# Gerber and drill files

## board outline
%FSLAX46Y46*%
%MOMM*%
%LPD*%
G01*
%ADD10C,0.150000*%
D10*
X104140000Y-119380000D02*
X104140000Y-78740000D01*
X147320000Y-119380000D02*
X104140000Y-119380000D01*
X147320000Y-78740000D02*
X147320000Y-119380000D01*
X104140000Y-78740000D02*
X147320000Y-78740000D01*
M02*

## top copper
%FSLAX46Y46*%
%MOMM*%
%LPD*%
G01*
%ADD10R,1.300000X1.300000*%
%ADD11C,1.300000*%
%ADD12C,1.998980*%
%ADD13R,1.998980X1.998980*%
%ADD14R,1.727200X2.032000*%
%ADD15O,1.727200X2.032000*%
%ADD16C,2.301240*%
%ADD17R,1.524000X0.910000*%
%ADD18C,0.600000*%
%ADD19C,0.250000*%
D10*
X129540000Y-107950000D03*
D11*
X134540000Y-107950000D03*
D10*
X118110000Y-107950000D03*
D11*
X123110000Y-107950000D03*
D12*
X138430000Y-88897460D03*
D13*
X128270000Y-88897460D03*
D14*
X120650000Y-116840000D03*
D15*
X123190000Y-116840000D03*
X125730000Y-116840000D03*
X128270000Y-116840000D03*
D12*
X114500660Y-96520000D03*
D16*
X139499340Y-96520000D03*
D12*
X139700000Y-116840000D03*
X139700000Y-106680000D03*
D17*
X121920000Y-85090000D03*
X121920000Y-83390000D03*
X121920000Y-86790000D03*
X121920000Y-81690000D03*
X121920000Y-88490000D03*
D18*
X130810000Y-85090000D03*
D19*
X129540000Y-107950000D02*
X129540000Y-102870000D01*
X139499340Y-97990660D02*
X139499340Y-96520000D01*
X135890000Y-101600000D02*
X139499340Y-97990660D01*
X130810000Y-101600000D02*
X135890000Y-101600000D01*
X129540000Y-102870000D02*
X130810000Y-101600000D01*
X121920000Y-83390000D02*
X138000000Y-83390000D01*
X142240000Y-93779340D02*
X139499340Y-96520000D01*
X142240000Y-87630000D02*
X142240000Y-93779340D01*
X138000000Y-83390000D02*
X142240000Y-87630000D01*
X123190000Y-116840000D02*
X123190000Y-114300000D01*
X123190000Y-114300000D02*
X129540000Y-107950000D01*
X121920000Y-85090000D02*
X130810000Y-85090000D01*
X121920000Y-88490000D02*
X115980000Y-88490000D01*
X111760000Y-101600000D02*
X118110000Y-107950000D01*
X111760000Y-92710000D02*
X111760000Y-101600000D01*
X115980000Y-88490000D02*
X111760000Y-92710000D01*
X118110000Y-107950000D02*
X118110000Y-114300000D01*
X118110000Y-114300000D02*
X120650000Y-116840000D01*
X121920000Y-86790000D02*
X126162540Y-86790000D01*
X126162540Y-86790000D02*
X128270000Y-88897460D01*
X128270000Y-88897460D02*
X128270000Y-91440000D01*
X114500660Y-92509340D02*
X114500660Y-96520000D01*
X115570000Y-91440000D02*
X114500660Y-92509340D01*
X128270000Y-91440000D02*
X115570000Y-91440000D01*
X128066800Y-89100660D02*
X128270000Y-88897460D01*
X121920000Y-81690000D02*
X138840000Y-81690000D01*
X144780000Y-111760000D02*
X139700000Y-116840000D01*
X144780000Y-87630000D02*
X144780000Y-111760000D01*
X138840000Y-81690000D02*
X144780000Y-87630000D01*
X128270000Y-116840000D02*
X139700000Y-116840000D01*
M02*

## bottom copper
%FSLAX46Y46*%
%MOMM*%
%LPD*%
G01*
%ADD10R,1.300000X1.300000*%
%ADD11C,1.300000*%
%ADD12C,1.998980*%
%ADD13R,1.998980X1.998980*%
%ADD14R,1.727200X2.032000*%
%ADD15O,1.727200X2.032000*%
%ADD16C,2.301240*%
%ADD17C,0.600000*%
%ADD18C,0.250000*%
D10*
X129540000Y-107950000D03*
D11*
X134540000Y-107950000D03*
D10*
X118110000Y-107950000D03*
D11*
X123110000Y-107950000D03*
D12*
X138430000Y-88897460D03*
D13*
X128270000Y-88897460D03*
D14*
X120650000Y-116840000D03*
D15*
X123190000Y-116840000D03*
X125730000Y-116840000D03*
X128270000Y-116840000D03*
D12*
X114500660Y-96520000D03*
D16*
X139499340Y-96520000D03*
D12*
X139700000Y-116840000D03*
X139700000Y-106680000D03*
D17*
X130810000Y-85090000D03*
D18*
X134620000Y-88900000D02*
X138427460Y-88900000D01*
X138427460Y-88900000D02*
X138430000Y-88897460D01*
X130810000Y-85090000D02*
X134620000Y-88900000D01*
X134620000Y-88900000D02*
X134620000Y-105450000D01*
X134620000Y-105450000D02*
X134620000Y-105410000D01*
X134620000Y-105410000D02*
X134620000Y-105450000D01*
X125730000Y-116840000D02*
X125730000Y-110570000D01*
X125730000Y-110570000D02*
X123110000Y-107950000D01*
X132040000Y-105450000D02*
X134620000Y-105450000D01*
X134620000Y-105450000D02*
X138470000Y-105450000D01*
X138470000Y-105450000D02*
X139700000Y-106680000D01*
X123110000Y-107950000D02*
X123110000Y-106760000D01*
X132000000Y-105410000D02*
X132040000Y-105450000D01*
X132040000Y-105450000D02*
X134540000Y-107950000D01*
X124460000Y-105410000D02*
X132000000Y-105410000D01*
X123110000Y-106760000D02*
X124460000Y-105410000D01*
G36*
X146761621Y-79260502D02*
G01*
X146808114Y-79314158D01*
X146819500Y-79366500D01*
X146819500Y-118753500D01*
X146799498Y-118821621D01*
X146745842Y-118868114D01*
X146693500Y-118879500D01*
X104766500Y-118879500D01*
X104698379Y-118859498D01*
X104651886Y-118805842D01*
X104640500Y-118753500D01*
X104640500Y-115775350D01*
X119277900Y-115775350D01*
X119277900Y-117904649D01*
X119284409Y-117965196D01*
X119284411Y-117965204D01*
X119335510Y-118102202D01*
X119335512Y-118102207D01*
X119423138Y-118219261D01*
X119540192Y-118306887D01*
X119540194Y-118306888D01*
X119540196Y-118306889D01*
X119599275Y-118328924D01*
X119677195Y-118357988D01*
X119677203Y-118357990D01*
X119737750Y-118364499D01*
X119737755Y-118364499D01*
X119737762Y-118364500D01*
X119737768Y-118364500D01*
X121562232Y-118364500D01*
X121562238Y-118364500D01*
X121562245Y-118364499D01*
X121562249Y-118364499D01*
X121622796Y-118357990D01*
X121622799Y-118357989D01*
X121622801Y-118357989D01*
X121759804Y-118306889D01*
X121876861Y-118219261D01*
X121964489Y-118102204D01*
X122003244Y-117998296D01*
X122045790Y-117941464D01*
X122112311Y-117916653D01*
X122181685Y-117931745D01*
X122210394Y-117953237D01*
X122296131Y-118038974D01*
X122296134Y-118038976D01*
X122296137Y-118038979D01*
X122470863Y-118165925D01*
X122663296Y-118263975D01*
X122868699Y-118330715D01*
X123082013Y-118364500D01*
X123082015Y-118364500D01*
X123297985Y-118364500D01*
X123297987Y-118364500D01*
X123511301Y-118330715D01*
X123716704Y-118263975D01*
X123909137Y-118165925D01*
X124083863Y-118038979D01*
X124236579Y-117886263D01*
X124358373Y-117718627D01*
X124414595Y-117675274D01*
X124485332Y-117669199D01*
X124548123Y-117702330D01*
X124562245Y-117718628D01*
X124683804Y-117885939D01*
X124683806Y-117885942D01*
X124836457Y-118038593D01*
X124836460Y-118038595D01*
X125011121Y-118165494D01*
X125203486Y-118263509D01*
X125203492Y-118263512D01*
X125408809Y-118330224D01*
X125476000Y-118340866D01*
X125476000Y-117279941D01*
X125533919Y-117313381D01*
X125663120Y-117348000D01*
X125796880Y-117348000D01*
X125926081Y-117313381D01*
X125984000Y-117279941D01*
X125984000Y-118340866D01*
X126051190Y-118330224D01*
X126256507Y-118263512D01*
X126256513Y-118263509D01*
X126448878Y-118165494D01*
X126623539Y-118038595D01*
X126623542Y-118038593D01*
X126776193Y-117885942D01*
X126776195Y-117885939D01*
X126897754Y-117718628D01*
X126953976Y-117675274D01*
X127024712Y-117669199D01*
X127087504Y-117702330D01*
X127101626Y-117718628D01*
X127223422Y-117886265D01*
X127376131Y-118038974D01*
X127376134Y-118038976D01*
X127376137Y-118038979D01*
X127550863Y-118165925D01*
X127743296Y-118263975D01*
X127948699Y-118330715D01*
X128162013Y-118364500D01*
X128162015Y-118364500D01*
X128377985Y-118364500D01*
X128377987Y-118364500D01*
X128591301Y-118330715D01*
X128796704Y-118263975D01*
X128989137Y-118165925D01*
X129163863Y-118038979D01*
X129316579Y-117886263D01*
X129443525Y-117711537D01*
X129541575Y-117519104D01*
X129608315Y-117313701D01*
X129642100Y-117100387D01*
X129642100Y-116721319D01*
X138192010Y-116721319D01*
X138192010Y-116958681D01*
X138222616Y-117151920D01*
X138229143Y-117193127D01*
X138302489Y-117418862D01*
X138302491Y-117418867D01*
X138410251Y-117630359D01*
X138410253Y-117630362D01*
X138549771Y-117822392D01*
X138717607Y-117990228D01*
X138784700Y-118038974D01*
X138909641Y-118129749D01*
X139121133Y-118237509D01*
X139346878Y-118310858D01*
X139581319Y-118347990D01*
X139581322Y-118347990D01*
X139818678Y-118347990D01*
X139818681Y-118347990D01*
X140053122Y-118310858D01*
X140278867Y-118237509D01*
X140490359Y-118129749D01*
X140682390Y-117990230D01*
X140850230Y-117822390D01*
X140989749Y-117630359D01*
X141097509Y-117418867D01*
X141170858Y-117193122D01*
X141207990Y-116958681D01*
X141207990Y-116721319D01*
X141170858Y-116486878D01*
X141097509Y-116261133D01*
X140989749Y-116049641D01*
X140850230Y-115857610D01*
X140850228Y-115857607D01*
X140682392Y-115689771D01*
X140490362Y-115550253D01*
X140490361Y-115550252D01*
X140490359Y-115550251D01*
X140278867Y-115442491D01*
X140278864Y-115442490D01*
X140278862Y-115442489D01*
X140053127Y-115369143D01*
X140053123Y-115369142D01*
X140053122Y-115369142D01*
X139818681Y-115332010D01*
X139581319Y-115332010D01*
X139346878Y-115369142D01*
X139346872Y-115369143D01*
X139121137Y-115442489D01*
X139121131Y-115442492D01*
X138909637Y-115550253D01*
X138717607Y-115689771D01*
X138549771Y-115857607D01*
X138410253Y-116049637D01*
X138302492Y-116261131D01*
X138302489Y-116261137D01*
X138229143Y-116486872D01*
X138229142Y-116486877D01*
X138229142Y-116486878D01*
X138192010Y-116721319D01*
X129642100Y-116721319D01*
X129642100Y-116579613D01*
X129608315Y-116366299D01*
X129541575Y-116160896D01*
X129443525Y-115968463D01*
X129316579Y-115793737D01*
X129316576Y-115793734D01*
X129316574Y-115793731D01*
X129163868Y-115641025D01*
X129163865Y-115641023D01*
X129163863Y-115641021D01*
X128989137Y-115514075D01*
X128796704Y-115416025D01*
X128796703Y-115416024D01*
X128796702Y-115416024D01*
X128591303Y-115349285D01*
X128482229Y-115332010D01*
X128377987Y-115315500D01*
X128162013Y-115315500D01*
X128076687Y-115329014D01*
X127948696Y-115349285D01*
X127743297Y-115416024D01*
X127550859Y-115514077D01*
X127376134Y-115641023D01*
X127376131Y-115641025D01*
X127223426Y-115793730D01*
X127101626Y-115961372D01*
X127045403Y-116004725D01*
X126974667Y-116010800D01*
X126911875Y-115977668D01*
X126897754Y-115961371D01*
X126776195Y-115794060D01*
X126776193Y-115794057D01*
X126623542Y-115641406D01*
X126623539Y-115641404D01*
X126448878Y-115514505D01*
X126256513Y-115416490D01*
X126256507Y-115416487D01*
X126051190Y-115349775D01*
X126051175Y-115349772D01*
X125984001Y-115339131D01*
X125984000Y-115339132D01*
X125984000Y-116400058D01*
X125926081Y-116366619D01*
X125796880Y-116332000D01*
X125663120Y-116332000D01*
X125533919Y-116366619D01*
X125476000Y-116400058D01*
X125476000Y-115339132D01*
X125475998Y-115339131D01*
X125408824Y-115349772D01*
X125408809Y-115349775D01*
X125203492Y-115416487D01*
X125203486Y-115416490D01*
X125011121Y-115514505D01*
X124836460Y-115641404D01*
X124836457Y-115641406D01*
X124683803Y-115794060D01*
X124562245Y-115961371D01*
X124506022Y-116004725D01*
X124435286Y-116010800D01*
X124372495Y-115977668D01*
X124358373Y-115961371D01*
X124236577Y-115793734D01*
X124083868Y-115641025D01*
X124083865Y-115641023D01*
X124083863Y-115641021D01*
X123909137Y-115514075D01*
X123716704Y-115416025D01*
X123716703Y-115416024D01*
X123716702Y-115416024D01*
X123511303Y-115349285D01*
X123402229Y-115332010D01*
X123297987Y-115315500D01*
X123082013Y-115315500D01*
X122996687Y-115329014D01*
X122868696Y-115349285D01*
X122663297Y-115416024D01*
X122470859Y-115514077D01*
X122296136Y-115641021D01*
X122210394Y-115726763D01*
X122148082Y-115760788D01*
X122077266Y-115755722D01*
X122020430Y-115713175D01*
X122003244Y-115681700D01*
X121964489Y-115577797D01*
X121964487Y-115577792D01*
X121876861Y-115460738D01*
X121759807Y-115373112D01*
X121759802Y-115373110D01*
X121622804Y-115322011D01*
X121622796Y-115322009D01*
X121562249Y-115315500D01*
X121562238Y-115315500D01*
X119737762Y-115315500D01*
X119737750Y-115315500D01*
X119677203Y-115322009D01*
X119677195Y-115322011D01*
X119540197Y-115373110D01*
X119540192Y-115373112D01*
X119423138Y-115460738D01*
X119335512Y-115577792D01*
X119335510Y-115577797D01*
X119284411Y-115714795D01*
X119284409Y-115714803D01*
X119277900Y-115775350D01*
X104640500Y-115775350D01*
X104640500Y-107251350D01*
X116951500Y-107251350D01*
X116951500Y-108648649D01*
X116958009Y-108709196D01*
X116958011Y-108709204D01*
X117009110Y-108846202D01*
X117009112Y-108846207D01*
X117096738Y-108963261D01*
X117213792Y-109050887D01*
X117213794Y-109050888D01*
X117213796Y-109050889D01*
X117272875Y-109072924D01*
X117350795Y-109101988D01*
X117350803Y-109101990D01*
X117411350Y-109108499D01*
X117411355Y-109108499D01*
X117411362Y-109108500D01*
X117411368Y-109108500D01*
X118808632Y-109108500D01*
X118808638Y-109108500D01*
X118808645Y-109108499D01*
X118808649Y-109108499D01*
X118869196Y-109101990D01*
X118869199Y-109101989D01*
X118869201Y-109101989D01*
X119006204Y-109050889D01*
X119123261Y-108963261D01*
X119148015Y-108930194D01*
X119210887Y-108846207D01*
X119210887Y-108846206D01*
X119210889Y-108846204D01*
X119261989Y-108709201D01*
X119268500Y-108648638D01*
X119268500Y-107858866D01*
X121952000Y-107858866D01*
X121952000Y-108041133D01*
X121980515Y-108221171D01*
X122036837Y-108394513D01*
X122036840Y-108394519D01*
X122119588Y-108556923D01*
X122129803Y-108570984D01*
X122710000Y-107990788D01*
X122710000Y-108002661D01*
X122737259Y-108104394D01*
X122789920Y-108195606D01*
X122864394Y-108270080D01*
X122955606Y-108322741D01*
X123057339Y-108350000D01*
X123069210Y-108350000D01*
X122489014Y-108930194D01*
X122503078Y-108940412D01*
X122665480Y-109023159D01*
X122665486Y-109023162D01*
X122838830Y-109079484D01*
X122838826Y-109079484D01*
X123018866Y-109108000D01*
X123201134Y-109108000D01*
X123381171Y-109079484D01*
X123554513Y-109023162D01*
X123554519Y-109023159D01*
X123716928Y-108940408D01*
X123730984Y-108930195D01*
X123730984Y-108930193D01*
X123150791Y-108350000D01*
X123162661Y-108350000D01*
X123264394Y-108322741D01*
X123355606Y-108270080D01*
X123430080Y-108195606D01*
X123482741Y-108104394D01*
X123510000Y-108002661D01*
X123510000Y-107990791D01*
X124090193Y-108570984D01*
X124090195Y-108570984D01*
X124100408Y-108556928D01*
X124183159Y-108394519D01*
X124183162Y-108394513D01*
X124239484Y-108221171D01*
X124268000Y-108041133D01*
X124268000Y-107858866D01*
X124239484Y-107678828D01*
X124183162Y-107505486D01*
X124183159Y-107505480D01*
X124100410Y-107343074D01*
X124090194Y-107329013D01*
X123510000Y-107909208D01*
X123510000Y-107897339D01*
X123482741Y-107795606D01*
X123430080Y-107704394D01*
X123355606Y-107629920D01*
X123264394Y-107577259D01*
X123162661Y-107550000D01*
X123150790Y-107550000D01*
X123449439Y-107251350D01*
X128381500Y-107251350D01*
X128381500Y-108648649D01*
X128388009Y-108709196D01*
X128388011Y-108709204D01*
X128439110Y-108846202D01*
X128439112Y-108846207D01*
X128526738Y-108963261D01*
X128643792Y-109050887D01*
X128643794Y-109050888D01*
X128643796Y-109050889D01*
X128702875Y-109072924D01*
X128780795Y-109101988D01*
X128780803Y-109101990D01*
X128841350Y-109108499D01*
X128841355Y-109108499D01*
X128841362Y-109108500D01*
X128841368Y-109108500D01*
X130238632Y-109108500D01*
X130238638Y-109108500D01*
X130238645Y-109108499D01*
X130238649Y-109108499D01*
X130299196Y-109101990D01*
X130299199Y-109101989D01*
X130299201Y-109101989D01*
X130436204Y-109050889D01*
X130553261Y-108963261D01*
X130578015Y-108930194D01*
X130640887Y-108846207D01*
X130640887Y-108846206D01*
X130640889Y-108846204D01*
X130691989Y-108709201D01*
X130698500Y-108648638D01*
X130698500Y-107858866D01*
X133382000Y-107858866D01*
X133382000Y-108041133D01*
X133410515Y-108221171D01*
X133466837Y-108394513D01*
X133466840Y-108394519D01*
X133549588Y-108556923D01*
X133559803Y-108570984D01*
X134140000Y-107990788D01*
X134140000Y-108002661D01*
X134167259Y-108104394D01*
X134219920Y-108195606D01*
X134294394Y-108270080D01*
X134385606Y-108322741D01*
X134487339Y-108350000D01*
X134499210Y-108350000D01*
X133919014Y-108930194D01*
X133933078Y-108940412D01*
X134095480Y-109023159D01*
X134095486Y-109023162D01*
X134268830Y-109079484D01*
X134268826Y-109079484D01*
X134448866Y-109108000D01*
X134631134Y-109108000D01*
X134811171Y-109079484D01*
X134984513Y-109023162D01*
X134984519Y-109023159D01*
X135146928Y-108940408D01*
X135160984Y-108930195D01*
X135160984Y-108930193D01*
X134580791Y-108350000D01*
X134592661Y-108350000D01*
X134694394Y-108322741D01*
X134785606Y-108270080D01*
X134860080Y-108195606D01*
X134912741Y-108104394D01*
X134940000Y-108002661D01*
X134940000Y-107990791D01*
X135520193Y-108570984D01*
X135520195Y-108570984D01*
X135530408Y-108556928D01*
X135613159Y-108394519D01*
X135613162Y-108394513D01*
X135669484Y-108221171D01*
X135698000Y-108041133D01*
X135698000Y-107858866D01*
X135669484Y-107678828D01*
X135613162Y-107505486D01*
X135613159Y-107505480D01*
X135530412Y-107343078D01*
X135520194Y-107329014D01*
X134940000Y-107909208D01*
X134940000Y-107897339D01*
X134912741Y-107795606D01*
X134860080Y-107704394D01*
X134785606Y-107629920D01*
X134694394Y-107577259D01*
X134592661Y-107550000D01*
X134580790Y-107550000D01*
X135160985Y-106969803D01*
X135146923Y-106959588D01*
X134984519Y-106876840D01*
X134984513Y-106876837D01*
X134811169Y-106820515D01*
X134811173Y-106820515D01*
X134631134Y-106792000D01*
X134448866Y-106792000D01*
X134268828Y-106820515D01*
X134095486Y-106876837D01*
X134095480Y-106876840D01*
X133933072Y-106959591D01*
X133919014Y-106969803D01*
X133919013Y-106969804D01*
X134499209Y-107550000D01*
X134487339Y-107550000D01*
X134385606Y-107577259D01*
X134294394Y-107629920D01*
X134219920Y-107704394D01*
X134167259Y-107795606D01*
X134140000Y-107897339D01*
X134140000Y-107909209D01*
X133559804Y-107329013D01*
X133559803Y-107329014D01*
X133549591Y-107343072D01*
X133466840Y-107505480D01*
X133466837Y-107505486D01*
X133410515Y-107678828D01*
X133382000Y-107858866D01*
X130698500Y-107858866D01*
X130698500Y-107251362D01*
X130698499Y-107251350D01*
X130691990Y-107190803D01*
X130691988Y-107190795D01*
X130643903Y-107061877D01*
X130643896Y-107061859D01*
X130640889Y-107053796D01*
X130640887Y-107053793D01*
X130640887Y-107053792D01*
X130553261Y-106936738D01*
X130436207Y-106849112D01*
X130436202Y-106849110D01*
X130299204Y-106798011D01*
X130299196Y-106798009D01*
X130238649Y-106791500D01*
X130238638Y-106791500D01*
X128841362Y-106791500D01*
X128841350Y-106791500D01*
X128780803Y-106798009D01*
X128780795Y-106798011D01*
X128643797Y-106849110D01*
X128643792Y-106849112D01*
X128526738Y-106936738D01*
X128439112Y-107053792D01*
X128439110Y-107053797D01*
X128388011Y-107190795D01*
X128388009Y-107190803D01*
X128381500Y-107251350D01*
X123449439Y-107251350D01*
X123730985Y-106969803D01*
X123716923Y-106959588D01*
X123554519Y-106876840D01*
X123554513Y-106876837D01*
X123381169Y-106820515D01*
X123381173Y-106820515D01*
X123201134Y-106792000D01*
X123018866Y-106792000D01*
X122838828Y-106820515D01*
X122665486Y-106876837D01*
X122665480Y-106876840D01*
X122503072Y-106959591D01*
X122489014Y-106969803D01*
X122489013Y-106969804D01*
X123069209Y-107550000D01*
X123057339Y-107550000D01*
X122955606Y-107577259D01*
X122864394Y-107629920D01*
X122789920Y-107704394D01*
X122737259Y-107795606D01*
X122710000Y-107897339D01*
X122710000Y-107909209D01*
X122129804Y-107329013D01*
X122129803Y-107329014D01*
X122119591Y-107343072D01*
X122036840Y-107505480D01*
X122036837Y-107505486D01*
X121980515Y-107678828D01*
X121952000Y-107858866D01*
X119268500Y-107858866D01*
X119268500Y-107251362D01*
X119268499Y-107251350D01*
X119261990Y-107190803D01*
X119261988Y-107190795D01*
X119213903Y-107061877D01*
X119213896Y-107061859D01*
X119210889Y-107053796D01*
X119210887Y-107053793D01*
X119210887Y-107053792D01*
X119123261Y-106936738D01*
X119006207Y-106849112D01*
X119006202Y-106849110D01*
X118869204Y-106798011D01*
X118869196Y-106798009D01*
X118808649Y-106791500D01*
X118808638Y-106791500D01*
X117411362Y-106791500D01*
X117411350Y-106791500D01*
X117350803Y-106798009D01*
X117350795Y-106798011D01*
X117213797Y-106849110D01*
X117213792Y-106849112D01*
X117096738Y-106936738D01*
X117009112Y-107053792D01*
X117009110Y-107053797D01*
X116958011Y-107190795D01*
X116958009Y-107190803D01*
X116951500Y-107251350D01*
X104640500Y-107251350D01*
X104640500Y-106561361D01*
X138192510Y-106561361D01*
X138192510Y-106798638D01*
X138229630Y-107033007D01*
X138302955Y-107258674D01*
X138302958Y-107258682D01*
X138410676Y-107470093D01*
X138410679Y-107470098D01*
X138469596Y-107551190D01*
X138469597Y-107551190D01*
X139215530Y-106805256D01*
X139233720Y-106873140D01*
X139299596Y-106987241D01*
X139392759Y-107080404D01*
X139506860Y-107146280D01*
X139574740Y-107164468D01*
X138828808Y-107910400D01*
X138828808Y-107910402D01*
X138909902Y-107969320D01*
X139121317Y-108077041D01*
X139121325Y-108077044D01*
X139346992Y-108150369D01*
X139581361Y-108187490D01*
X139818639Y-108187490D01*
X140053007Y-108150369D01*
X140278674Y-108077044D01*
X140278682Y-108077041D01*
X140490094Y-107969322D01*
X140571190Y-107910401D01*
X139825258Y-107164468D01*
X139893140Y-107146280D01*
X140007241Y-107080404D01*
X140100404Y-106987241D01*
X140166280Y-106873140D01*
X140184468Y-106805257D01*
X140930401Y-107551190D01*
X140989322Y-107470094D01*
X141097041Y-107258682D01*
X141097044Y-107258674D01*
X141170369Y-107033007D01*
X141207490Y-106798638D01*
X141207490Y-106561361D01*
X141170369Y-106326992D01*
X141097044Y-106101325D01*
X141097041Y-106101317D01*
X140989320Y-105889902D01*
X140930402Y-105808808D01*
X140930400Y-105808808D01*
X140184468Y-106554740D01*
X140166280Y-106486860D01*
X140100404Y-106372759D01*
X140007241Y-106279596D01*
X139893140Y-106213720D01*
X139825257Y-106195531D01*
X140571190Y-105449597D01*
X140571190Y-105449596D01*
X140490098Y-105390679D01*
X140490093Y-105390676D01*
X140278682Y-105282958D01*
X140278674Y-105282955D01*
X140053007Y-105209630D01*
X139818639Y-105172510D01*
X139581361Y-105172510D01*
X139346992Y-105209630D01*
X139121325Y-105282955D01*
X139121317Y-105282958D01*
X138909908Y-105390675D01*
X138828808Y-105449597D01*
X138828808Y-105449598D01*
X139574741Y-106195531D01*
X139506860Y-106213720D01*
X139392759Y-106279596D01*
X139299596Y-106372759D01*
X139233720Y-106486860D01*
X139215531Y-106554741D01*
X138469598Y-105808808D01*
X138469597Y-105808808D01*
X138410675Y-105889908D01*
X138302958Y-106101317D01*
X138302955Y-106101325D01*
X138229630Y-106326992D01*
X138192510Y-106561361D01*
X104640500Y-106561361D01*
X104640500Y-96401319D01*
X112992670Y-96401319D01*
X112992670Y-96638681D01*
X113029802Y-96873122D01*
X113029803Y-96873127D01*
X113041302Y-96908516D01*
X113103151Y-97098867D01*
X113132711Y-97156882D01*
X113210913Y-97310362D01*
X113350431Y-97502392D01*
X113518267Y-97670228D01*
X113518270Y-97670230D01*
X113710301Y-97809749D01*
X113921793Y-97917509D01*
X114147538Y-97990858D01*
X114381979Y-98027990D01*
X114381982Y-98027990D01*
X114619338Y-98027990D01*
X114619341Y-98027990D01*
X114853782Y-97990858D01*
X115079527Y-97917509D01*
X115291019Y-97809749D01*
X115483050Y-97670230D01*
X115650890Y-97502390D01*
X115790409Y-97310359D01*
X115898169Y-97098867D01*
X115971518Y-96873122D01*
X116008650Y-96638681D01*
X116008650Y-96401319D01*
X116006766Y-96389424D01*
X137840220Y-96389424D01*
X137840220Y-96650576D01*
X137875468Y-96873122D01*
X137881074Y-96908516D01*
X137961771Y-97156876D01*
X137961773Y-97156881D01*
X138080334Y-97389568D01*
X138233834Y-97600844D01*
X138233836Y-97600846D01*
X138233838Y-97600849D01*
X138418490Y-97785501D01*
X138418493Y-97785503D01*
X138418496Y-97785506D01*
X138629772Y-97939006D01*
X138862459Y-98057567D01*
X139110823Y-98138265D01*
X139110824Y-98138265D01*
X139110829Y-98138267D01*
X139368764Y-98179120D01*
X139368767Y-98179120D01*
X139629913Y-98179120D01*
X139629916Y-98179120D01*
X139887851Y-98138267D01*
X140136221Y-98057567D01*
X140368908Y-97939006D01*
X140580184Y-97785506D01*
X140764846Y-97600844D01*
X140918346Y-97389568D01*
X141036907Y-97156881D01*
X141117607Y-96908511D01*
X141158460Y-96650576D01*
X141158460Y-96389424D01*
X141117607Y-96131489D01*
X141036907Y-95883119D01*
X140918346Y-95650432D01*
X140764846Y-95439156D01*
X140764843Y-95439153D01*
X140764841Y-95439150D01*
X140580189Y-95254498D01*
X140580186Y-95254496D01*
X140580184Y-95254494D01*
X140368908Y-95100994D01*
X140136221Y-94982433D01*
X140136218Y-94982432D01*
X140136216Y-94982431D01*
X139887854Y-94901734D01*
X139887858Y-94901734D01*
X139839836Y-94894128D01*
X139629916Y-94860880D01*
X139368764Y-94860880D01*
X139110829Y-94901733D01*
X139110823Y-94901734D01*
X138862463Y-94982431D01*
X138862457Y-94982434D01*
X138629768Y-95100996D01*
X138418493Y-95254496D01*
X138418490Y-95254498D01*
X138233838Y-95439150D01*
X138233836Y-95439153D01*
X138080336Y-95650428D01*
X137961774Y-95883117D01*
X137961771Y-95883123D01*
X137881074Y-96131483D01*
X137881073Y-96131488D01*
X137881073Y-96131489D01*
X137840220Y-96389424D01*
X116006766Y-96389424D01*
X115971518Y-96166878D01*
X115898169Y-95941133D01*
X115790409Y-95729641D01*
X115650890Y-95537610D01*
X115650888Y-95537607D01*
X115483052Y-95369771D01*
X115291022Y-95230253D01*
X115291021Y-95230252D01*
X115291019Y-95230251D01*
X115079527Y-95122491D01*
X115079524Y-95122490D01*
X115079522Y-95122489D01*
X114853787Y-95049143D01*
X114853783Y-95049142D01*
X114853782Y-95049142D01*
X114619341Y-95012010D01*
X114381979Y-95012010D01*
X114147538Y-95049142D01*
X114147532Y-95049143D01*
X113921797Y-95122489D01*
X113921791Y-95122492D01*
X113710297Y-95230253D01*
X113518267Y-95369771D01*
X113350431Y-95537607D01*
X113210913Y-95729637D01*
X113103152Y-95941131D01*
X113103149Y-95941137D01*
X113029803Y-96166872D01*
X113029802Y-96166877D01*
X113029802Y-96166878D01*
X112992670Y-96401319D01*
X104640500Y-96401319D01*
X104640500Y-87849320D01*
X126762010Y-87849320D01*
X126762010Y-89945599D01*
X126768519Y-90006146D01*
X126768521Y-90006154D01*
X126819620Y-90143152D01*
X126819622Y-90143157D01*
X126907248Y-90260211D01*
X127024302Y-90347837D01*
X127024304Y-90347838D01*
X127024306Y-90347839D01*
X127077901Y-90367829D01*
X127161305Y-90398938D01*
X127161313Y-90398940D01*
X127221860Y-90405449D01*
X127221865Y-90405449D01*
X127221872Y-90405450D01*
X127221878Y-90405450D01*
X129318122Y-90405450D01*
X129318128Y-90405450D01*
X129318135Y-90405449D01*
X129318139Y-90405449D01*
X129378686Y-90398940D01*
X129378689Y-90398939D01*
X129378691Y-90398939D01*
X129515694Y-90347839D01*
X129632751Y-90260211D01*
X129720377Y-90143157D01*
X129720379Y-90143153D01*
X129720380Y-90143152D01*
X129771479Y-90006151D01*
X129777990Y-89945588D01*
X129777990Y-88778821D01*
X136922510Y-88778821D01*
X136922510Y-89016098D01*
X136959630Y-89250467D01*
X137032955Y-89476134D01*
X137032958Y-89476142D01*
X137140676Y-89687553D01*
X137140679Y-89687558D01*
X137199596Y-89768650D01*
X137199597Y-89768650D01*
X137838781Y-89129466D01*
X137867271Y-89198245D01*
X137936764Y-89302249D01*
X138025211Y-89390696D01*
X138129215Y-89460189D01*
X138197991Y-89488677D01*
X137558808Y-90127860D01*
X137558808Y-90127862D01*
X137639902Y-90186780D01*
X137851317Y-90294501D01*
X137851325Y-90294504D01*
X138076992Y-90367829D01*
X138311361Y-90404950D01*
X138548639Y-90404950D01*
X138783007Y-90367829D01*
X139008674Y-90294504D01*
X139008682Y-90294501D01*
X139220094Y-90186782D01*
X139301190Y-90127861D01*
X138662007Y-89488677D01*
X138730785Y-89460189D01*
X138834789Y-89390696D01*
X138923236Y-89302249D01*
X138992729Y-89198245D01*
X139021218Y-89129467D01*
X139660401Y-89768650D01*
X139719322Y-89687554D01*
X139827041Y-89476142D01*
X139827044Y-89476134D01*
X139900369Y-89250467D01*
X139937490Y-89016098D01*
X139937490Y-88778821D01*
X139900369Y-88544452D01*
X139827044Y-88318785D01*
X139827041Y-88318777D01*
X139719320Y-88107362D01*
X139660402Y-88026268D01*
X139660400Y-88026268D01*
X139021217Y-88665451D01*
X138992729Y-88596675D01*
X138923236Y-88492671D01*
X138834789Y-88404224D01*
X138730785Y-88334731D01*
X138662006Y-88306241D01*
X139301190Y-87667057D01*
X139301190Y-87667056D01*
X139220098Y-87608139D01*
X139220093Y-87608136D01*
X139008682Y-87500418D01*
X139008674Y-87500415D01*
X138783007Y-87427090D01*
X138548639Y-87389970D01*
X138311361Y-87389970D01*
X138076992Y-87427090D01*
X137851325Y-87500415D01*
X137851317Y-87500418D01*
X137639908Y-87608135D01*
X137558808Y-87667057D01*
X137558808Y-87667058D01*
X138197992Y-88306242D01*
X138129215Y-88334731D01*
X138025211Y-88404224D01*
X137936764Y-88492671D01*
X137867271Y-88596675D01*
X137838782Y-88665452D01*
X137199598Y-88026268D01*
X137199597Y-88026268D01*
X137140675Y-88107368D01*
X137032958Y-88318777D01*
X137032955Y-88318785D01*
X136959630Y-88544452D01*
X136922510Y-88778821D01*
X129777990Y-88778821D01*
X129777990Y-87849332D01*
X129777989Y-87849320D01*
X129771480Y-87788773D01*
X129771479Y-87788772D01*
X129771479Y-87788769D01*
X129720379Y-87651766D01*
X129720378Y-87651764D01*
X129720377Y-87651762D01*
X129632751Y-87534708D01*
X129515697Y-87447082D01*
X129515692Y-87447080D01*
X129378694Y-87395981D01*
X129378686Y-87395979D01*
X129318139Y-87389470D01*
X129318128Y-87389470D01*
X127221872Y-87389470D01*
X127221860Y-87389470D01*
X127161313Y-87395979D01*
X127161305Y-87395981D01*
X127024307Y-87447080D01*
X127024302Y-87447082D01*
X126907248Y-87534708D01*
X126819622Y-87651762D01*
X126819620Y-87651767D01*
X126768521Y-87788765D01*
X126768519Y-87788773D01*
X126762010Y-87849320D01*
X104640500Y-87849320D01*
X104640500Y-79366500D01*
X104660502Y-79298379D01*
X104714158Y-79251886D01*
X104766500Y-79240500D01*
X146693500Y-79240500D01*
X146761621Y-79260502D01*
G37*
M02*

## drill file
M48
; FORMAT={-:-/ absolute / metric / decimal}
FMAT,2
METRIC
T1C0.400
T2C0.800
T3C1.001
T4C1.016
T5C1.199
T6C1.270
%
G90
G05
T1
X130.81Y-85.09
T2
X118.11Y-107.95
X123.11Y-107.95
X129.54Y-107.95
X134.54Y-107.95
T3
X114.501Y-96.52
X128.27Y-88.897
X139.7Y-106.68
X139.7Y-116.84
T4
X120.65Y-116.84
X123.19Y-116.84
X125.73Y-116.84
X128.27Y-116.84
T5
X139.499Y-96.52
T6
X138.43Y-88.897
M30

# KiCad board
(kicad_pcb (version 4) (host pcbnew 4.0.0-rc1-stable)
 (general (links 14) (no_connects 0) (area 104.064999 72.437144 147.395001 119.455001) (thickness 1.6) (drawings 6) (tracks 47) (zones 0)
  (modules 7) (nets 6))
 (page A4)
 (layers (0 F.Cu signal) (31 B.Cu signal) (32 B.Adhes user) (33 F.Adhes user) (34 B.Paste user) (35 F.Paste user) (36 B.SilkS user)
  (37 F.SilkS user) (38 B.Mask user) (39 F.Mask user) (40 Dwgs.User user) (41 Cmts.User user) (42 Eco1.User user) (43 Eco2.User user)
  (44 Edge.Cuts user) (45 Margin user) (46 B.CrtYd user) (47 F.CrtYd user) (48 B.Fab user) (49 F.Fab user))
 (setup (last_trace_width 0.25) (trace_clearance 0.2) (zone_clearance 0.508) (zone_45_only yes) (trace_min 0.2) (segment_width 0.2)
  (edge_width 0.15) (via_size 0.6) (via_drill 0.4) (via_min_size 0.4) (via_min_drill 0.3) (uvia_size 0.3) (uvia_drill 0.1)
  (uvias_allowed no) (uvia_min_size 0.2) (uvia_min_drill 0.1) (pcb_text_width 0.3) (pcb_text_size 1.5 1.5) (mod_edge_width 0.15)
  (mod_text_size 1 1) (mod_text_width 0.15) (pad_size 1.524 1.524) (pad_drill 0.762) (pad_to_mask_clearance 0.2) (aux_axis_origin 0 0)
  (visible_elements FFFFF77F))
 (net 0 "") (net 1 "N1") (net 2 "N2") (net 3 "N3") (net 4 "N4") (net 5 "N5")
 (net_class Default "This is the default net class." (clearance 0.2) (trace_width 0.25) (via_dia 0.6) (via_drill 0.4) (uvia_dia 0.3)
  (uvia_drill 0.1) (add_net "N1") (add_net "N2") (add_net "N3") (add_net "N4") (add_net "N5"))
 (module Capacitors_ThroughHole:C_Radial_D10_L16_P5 (layer F.Cu) (at 129.54 107.95)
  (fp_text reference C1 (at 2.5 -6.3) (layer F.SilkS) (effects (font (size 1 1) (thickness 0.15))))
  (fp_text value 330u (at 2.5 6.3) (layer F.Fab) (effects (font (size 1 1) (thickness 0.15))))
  (pad 1 thru_hole rect (at 0 0) (size 1.3 1.3) (drill 0.8) (layers *.Cu *.Mask F.SilkS) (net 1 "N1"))
  (pad 2 thru_hole circle (at 5 0) (size 1.3 1.3) (drill 0.8) (layers *.Cu *.Mask F.SilkS) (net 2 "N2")))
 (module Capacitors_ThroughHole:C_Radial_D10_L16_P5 (layer F.Cu) (at 118.11 107.95)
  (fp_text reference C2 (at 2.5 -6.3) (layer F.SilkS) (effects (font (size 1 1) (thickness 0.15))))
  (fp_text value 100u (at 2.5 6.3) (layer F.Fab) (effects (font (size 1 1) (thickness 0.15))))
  (pad 1 thru_hole rect (at 0 0) (size 1.3 1.3) (drill 0.8) (layers *.Cu *.Mask F.SilkS) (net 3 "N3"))
  (pad 2 thru_hole circle (at 5 0) (size 1.3 1.3) (drill 0.8) (layers *.Cu *.Mask F.SilkS) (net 2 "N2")))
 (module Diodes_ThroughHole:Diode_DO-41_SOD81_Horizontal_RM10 (layer F.Cu) (at 128.27 88.9)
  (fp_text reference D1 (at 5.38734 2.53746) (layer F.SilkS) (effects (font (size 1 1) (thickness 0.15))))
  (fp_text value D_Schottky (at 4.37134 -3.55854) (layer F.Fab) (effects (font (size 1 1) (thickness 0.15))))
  (pad 2 thru_hole circle (at 10.16 -0.00254 180) (size 1.99898 1.99898) (drill 1.27) (layers *.Cu *.Mask F.SilkS) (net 2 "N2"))
  (pad 1 thru_hole rect (at 0 -0.00254 180) (size 1.99898 1.99898) (drill 1.00076) (layers *.Cu *.Mask F.SilkS) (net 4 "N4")))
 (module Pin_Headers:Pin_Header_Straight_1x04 (layer F.Cu) (at 120.65 116.84 90)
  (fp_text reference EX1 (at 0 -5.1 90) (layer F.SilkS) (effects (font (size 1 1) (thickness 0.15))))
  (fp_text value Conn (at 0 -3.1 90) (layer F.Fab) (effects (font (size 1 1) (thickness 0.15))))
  (pad 1 thru_hole rect (at 0 0 90) (size 2.032 1.7272) (drill 1.016) (layers *.Cu *.Mask F.SilkS) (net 3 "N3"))
  (pad 2 thru_hole oval (at 0 2.54 90) (size 2.032 1.7272) (drill 1.016) (layers *.Cu *.Mask F.SilkS) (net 1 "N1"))
  (pad 3 thru_hole oval (at 0 5.08 90) (size 2.032 1.7272) (drill 1.016) (layers *.Cu *.Mask F.SilkS) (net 2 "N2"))
  (pad 4 thru_hole oval (at 0 7.62 90) (size 2.032 1.7272) (drill 1.016) (layers *.Cu *.Mask F.SilkS) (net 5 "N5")))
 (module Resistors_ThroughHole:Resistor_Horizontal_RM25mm (layer F.Cu) (at 127 96.52)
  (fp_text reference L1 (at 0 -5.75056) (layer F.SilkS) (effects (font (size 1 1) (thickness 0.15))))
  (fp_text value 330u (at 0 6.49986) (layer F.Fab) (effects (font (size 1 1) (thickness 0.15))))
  (pad 1 thru_hole circle (at -12.49934 0) (size 1.99898 1.99898) (drill 1.00076) (layers *.Cu *.SilkS *.Mask) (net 4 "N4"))
  (pad 2 thru_hole circle (at 12.49934 0) (size 2.30124 2.30124) (drill 1.19888) (layers *.Cu *.SilkS *.Mask) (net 1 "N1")))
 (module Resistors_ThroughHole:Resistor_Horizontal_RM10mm (layer F.Cu) (at 139.7 111.76 90)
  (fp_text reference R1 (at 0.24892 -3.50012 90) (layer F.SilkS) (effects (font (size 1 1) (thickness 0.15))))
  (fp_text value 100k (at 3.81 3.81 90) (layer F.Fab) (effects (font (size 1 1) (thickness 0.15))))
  (pad 1 thru_hole circle (at -5.08 0 90) (size 1.99898 1.99898) (drill 1.00076) (layers *.Cu *.SilkS *.Mask) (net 5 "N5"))
  (pad 2 thru_hole circle (at 5.08 0 90) (size 1.99898 1.99898) (drill 1.00076) (layers *.Cu *.SilkS *.Mask) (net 2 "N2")))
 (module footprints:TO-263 (layer F.Cu) (at 121.92 85.09 90)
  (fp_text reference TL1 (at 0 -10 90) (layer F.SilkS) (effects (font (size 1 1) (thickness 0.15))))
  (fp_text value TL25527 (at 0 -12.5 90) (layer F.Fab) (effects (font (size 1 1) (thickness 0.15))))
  (pad 3 smd rect (at 0 0 90) (size 0.91 1.524) (layers F.Cu F.Paste F.Mask) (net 2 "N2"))
  (pad 4 smd rect (at 1.7 0 90) (size 0.91 1.524) (layers F.Cu F.Paste F.Mask) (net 1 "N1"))
  (pad 2 smd rect (at -1.7 0 90) (size 0.91 1.524) (layers F.Cu F.Paste F.Mask) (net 4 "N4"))
  (pad 5 smd rect (at 3.4 0 90) (size 0.91 1.524) (layers F.Cu F.Paste F.Mask) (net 5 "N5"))
  (pad 1 smd rect (at -3.4 0 90) (size 0.91 1.524) (layers F.Cu F.Paste F.Mask) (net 3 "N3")))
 (gr_line (start 104.14 119.38) (end 104.14 78.74) (angle 90) (layer Edge.Cuts) (width 0.15))
 (gr_line (start 147.32 119.38) (end 104.14 119.38) (angle 90) (layer Edge.Cuts) (width 0.15))
 (gr_line (start 147.32 78.74) (end 147.32 119.38) (angle 90) (layer Edge.Cuts) (width 0.15))
 (gr_line (start 104.14 78.74) (end 147.32 78.74) (angle 90) (layer Edge.Cuts) (width 0.15))
 (segment (start 129.54 107.95) (end 129.54 102.87) (width 0.25) (layer F.Cu) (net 1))
 (segment (start 139.49934 97.99066) (end 139.49934 96.52) (width 0.25) (layer F.Cu) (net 1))
 (segment (start 135.89 101.6) (end 139.49934 97.99066) (width 0.25) (layer F.Cu) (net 1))
 (segment (start 130.81 101.6) (end 135.89 101.6) (width 0.25) (layer F.Cu) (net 1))
 (segment (start 129.54 102.87) (end 130.81 101.6) (width 0.25) (layer F.Cu) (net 1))
 (segment (start 121.92 83.39) (end 138 83.39) (width 0.25) (layer F.Cu) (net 1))
 (segment (start 142.24 93.77934) (end 139.49934 96.52) (width 0.25) (layer F.Cu) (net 1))
 (segment (start 142.24 87.63) (end 142.24 93.77934) (width 0.25) (layer F.Cu) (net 1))
 (segment (start 138 83.39) (end 142.24 87.63) (width 0.25) (layer F.Cu) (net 1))
 (segment (start 123.19 116.84) (end 123.19 114.3) (width 0.25) (layer F.Cu) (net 1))
 (segment (start 123.19 114.3) (end 129.54 107.95) (width 0.25) (layer F.Cu) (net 1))
 (segment (start 134.62 88.9) (end 138.42746 88.9) (width 0.25) (layer B.Cu) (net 2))
 (segment (start 138.42746 88.9) (end 138.43 88.89746) (width 0.25) (layer B.Cu) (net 2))
 (segment (start 121.92 85.09) (end 130.81 85.09) (width 0.25) (layer F.Cu) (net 2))
 (via (at 130.81 85.09) (size 0.6) (drill 0.4) (layers F.Cu B.Cu) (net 2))
 (segment (start 130.81 85.09) (end 134.62 88.9) (width 0.25) (layer B.Cu) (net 2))
 (segment (start 134.62 88.9) (end 134.62 105.45) (width 0.25) (layer B.Cu) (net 2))
 (segment (start 134.62 105.45) (end 134.62 105.41) (width 0.25) (layer B.Cu) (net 2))
 (segment (start 134.62 105.41) (end 134.62 105.45) (width 0.25) (layer B.Cu) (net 2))
 (segment (start 125.73 116.84) (end 125.73 110.57) (width 0.25) (layer B.Cu) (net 2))
 (segment (start 125.73 110.57) (end 123.11 107.95) (width 0.25) (layer B.Cu) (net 2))
 (segment (start 132.04 105.45) (end 134.62 105.45) (width 0.25) (layer B.Cu) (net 2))
 (segment (start 134.62 105.45) (end 138.47 105.45) (width 0.25) (layer B.Cu) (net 2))
 (segment (start 138.47 105.45) (end 139.7 106.68) (width 0.25) (layer B.Cu) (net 2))
 (segment (start 123.11 107.95) (end 123.11 106.76) (width 0.25) (layer B.Cu) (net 2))
 (segment (start 132 105.41) (end 132.04 105.45) (width 0.25) (layer B.Cu) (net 2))
 (segment (start 132.04 105.45) (end 134.54 107.95) (width 0.25) (layer B.Cu) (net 2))
 (segment (start 124.46 105.41) (end 132 105.41) (width 0.25) (layer B.Cu) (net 2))
 (segment (start 123.11 106.76) (end 124.46 105.41) (width 0.25) (layer B.Cu) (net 2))
 (segment (start 121.92 88.49) (end 115.98 88.49) (width 0.25) (layer F.Cu) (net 3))
 (segment (start 111.76 101.6) (end 118.11 107.95) (width 0.25) (layer F.Cu) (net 3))
 (segment (start 111.76 92.71) (end 111.76 101.6) (width 0.25) (layer F.Cu) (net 3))
 (segment (start 115.98 88.49) (end 111.76 92.71) (width 0.25) (layer F.Cu) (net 3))
 (segment (start 118.11 107.95) (end 118.11 114.3) (width 0.25) (layer F.Cu) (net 3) (status 10))
 (segment (start 118.11 114.3) (end 120.65 116.84) (width 0.25) (layer F.Cu) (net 3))
 (segment (start 121.92 86.79) (end 126.16254 86.79) (width 0.25) (layer F.Cu) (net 4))
 (segment (start 126.16254 86.79) (end 128.27 88.89746) (width 0.25) (layer F.Cu) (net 4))
 (segment (start 128.27 88.89746) (end 128.27 91.44) (width 0.25) (layer F.Cu) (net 4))
 (segment (start 114.50066 92.50934) (end 114.50066 96.52) (width 0.25) (layer F.Cu) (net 4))
 (segment (start 115.57 91.44) (end 114.50066 92.50934) (width 0.25) (layer F.Cu) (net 4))
 (segment (start 128.27 91.44) (end 115.57 91.44) (width 0.25) (layer F.Cu) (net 4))
 (segment (start 128.0668 89.10066) (end 128.27 88.89746) (width 0.25) (layer F.Cu) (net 4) (status 30))
 (segment (start 121.92 81.69) (end 138.84 81.69) (width 0.25) (layer F.Cu) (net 5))
 (segment (start 144.78 111.76) (end 139.7 116.84) (width 0.25) (layer F.Cu) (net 5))
 (segment (start 144.78 87.63) (end 144.78 111.76) (width 0.25) (layer F.Cu) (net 5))
 (segment (start 138.84 81.69) (end 144.78 87.63) (width 0.25) (layer F.Cu) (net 5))
 (segment (start 128.27 116.84) (end 139.7 116.84) (width 0.25) (layer F.Cu) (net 5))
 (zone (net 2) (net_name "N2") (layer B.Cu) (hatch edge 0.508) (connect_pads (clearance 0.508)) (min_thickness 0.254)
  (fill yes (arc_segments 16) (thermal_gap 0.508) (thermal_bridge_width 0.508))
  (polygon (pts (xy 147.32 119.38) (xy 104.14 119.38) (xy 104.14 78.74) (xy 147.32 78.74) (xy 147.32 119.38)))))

